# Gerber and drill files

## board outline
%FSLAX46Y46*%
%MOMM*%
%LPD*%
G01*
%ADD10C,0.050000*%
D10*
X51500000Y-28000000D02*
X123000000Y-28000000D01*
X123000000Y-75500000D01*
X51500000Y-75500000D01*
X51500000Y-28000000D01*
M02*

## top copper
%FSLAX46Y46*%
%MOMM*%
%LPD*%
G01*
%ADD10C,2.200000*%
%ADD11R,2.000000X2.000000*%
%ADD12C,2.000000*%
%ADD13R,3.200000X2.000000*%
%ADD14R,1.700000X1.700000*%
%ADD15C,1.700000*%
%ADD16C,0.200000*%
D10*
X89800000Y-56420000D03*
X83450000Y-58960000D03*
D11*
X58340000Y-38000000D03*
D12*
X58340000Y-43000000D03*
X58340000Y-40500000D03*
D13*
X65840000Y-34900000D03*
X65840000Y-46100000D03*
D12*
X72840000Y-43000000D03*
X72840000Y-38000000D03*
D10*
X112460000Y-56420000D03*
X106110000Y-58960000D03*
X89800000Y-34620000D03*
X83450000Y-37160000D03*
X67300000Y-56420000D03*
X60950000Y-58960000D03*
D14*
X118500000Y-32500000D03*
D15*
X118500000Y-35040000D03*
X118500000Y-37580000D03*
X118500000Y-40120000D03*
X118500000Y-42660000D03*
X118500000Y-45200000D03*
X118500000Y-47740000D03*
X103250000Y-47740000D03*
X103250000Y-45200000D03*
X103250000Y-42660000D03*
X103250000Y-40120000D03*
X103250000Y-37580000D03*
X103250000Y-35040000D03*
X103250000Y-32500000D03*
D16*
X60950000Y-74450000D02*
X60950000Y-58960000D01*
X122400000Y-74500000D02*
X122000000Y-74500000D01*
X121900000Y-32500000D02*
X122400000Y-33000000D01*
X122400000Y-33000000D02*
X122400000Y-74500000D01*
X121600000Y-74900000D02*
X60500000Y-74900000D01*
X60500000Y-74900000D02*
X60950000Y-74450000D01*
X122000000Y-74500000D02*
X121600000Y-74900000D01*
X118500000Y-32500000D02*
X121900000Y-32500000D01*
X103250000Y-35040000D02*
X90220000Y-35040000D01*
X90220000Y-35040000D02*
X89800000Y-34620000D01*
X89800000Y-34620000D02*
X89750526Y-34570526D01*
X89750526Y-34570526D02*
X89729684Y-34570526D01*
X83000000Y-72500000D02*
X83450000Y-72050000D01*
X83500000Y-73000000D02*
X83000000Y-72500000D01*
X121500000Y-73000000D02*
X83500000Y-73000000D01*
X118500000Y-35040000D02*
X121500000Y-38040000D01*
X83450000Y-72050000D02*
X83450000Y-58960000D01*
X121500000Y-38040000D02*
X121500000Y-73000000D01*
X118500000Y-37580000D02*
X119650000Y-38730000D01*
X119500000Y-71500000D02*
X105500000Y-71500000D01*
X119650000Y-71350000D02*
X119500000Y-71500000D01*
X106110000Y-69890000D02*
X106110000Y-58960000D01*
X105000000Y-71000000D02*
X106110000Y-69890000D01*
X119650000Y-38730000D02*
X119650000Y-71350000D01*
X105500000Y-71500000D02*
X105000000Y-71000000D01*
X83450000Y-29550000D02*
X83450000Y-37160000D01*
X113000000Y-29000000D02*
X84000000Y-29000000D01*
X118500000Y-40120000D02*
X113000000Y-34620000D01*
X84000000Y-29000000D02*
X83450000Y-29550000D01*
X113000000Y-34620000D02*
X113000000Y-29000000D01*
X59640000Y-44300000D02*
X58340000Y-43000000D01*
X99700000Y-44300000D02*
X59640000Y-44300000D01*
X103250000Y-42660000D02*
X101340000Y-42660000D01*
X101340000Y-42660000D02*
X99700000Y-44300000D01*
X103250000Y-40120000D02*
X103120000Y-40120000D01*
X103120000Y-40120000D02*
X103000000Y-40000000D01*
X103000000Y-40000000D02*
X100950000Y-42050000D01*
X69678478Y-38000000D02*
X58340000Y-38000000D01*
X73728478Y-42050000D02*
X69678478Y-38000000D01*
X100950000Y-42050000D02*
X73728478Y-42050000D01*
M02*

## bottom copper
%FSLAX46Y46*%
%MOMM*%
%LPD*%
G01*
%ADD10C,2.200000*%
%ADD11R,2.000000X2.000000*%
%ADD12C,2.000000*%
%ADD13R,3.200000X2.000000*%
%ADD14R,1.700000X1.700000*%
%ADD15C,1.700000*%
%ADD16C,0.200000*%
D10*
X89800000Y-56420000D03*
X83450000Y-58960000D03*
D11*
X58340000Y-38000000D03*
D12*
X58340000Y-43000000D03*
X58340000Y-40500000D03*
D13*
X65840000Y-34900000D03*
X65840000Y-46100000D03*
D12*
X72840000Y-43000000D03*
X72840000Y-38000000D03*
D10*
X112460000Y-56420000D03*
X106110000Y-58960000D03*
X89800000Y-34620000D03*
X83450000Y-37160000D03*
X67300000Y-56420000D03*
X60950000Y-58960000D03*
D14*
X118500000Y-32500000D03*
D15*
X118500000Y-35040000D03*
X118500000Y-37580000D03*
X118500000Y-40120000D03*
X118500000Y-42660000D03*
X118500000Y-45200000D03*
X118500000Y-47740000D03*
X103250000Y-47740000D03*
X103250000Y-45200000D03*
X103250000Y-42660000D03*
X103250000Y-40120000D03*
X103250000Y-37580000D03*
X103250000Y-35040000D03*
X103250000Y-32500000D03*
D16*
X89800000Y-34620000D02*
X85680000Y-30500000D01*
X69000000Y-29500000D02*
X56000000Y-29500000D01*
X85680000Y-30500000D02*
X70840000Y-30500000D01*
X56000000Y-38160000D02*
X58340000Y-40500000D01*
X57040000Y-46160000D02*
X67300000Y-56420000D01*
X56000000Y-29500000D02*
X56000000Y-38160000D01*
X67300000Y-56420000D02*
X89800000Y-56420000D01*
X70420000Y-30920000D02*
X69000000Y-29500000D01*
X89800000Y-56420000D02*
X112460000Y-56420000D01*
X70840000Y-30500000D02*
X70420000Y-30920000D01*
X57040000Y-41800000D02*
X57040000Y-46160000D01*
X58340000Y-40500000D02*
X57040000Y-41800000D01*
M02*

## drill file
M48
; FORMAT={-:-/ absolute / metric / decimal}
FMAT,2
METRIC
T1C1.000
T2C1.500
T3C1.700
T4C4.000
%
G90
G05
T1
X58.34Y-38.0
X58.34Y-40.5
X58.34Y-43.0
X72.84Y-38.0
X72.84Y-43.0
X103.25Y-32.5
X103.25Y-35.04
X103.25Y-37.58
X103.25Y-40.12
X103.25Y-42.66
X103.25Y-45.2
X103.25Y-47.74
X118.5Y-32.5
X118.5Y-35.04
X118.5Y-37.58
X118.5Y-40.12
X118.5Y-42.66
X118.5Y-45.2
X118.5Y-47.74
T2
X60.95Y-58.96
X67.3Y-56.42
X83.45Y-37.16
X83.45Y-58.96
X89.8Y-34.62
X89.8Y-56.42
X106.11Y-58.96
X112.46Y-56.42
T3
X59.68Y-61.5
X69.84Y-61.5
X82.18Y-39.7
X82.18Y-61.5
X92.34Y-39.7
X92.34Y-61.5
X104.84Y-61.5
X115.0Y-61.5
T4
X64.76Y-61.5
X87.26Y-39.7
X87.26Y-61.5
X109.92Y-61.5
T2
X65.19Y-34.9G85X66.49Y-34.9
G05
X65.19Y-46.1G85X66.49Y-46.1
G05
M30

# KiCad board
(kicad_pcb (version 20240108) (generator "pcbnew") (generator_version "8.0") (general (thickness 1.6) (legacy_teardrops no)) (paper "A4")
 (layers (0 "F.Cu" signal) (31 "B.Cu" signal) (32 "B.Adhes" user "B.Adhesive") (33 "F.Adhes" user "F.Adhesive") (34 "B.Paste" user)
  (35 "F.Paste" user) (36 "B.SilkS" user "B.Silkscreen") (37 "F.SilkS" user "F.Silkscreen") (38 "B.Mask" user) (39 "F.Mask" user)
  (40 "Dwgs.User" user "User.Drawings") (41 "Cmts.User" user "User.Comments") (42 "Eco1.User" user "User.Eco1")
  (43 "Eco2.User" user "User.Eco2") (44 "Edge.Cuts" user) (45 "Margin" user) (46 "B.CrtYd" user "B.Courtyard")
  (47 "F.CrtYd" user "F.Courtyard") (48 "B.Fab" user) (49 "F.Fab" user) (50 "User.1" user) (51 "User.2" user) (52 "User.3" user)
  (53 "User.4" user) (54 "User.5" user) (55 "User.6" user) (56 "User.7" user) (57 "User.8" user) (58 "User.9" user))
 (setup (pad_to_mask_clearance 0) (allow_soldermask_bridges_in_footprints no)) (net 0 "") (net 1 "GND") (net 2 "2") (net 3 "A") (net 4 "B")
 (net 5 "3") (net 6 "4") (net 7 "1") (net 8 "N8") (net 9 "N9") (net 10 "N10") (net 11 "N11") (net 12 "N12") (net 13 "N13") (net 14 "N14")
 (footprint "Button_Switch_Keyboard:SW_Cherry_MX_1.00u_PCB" (layer "F.Cu") (at 89.8 56.42)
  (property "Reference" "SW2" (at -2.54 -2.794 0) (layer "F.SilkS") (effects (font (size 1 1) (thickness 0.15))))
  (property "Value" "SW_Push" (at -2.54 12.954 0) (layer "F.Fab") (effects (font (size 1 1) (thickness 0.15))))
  (pad "" np_thru_hole circle (at -7.62 5.08) (size 1.7 1.7) (drill 1.7) (layers "*.Cu" "*.Mask"))
  (pad "" np_thru_hole circle (at -2.54 5.08) (size 4 4) (drill 4) (layers "*.Cu" "*.Mask"))
  (pad "" np_thru_hole circle (at 2.54 5.08) (size 1.7 1.7) (drill 1.7) (layers "*.Cu" "*.Mask"))
  (pad "1" thru_hole circle (at 0 0) (size 2.2 2.2) (drill 1.5) (layers "*.Cu" "*.Mask") (remove_unused_layers no) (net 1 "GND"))
  (pad "2" thru_hole circle (at -6.35 2.54) (size 2.2 2.2) (drill 1.5) (layers "*.Cu" "*.Mask") (remove_unused_layers no) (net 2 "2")))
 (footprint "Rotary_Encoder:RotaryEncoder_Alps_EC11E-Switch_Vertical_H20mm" (layer "F.Cu") (at 58.34 38)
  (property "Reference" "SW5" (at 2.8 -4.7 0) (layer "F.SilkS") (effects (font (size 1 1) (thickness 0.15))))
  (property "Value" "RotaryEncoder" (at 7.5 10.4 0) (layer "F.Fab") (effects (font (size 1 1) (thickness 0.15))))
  (pad "A" thru_hole rect (at 0 0) (size 2 2) (drill 1) (layers "*.Cu" "*.Mask") (remove_unused_layers no) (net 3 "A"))
  (pad "B" thru_hole circle (at 0 5) (size 2 2) (drill 1) (layers "*.Cu" "*.Mask") (remove_unused_layers no) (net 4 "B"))
  (pad "C" thru_hole circle (at 0 2.5) (size 2 2) (drill 1) (layers "*.Cu" "*.Mask") (remove_unused_layers no) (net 1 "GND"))
  (pad "MP" thru_hole rect (at 7.5 -3.1) (size 3.2 2) (drill oval 2.8 1.5) (layers "*.Cu" "*.Mask") (remove_unused_layers no))
  (pad "MP" thru_hole rect (at 7.5 8.1) (size 3.2 2) (drill oval 2.8 1.5) (layers "*.Cu" "*.Mask") (remove_unused_layers no))
  (pad "S1" thru_hole circle (at 14.5 5) (size 2 2) (drill 1) (layers "*.Cu" "*.Mask") (remove_unused_layers no))
  (pad "S2" thru_hole circle (at 14.5 0) (size 2 2) (drill 1) (layers "*.Cu" "*.Mask") (remove_unused_layers no)))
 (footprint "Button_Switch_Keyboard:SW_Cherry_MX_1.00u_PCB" (layer "F.Cu") (at 112.46 56.42)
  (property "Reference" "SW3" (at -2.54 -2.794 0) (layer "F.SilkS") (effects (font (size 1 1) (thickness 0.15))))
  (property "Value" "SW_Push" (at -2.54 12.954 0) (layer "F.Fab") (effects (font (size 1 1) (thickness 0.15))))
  (pad "" np_thru_hole circle (at -7.62 5.08) (size 1.7 1.7) (drill 1.7) (layers "*.Cu" "*.Mask"))
  (pad "" np_thru_hole circle (at -2.54 5.08) (size 4 4) (drill 4) (layers "*.Cu" "*.Mask"))
  (pad "" np_thru_hole circle (at 2.54 5.08) (size 1.7 1.7) (drill 1.7) (layers "*.Cu" "*.Mask"))
  (pad "1" thru_hole circle (at 0 0) (size 2.2 2.2) (drill 1.5) (layers "*.Cu" "*.Mask") (remove_unused_layers no) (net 1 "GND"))
  (pad "2" thru_hole circle (at -6.35 2.54) (size 2.2 2.2) (drill 1.5) (layers "*.Cu" "*.Mask") (remove_unused_layers no) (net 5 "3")))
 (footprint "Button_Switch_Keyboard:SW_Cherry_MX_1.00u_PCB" (layer "F.Cu") (at 89.8 34.62)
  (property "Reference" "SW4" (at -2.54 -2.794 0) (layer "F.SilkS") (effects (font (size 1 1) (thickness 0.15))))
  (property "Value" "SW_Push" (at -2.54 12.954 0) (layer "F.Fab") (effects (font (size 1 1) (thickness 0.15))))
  (pad "" np_thru_hole circle (at -7.62 5.08) (size 1.7 1.7) (drill 1.7) (layers "*.Cu" "*.Mask"))
  (pad "" np_thru_hole circle (at -2.54 5.08) (size 4 4) (drill 4) (layers "*.Cu" "*.Mask"))
  (pad "" np_thru_hole circle (at 2.54 5.08) (size 1.7 1.7) (drill 1.7) (layers "*.Cu" "*.Mask"))
  (pad "1" thru_hole circle (at 0 0) (size 2.2 2.2) (drill 1.5) (layers "*.Cu" "*.Mask") (remove_unused_layers no) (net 1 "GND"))
  (pad "2" thru_hole circle (at -6.35 2.54) (size 2.2 2.2) (drill 1.5) (layers "*.Cu" "*.Mask") (remove_unused_layers no) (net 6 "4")))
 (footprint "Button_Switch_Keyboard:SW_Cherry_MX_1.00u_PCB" (layer "F.Cu") (at 67.3 56.42)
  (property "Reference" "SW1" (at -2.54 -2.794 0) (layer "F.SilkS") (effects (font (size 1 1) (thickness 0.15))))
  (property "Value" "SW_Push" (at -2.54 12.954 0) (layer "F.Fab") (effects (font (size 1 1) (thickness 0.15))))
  (pad "" np_thru_hole circle (at -7.62 5.08) (size 1.7 1.7) (drill 1.7) (layers "*.Cu" "*.Mask"))
  (pad "" np_thru_hole circle (at -2.54 5.08) (size 4 4) (drill 4) (layers "*.Cu" "*.Mask"))
  (pad "" np_thru_hole circle (at 2.54 5.08) (size 1.7 1.7) (drill 1.7) (layers "*.Cu" "*.Mask"))
  (pad "1" thru_hole circle (at 0 0) (size 2.2 2.2) (drill 1.5) (layers "*.Cu" "*.Mask") (remove_unused_layers no) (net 1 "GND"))
  (pad "2" thru_hole circle (at -6.35 2.54) (size 2.2 2.2) (drill 1.5) (layers "*.Cu" "*.Mask") (remove_unused_layers no) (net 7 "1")))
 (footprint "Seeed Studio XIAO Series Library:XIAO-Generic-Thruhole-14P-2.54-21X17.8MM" (layer "B.Cu") (at 110.875 40.12 180)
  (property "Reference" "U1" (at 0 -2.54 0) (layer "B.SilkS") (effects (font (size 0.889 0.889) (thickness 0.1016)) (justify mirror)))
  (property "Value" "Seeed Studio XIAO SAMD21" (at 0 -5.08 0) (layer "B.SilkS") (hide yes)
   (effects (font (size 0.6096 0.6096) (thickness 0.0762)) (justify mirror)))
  (pad "1" thru_hole rect (at -7.625 7.62 180) (size 1.7 1.7) (drill 1) (layers "*.Cu" "*.Mask") (remove_unused_layers no) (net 7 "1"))
  (pad "2" thru_hole circle (at -7.625 5.08 180) (size 1.7 1.7) (drill 1) (layers "*.Cu" "*.Mask") (remove_unused_layers no) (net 2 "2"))
  (pad "3" thru_hole circle (at -7.625 2.54 180) (size 1.7 1.7) (drill 1) (layers "*.Cu" "*.Mask") (remove_unused_layers no) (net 5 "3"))
  (pad "4" thru_hole circle (at -7.625 0 180) (size 1.7 1.7) (drill 1) (layers "*.Cu" "*.Mask") (remove_unused_layers no) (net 6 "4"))
  (pad "5" thru_hole circle (at -7.625 -2.54 180) (size 1.7 1.7) (drill 1) (layers "*.Cu" "*.Mask") (remove_unused_layers no) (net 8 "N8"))
  (pad "6" thru_hole circle (at -7.625 -5.08) (size 1.7 1.7) (drill 1) (layers "*.Cu" "*.Mask") (remove_unused_layers no) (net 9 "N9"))
  (pad "7" thru_hole circle (at -7.625 -7.62 180) (size 1.7 1.7) (drill 1) (layers "*.Cu" "*.Mask") (remove_unused_layers no) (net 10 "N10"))
  (pad "8" thru_hole circle (at 7.625 -7.62 180) (size 1.7 1.7) (drill 1) (layers "*.Cu" "*.Mask") (remove_unused_layers no) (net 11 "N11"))
  (pad "9" thru_hole circle (at 7.625 -5.08 180) (size 1.7 1.7) (drill 1) (layers "*.Cu" "*.Mask") (remove_unused_layers no) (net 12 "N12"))
  (pad "10" thru_hole circle (at 7.625 -2.54 180) (size 1.7 1.7) (drill 1) (layers "*.Cu" "*.Mask") (remove_unused_layers no) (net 4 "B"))
  (pad "11" thru_hole circle (at 7.625 0 180) (size 1.7 1.7) (drill 1) (layers "*.Cu" "*.Mask") (remove_unused_layers no) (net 3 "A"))
  (pad "12" thru_hole circle (at 7.625 2.54 180) (size 1.7 1.7) (drill 1) (layers "*.Cu" "*.Mask") (remove_unused_layers no) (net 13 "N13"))
  (pad "13" thru_hole circle (at 7.625 5.08 180) (size 1.7 1.7) (drill 1) (layers "*.Cu" "*.Mask") (remove_unused_layers no) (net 1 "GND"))
  (pad "14" thru_hole circle (at 7.625 7.62 180) (size 1.7 1.7) (drill 1) (layers "*.Cu" "*.Mask") (remove_unused_layers no) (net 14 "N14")))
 (gr_rect (start 51.5 28) (end 123 75.5) (stroke (width 0.05) (type default)) (fill none) (layer "Edge.Cuts"))
 (segment (start 60.95 74.45) (end 60.95 58.96) (width 0.2) (layer "F.Cu") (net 7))
 (segment (start 122.4 74.5) (end 122 74.5) (width 0.2) (layer "F.Cu") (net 7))
 (segment (start 121.9 32.5) (end 122.4 33) (width 0.2) (layer "F.Cu") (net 7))
 (segment (start 122.4 33) (end 122.4 74.5) (width 0.2) (layer "F.Cu") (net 7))
 (segment (start 121.6 74.9) (end 60.5 74.9) (width 0.2) (layer "F.Cu") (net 7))
 (segment (start 60.5 74.9) (end 60.95 74.45) (width 0.2) (layer "F.Cu") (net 7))
 (segment (start 122 74.5) (end 121.6 74.9) (width 0.2) (layer "F.Cu") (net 7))
 (segment (start 118.5 32.5) (end 121.9 32.5) (width 0.2) (layer "F.Cu") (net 7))
 (segment (start 103.25 35.04) (end 90.22 35.04) (width 0.2) (layer "F.Cu") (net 1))
 (segment (start 90.22 35.04) (end 89.8 34.62) (width 0.2) (layer "F.Cu") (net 1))
 (segment (start 89.8 34.62) (end 89.750526 34.570526) (width 0.2) (layer "F.Cu") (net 1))
 (segment (start 89.750526 34.570526) (end 89.729684 34.570526) (width 0.2) (layer "F.Cu") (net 1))
 (segment (start 89.8 34.62) (end 85.68 30.5) (width 0.2) (layer "B.Cu") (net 1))
 (segment (start 69 29.5) (end 56 29.5) (width 0.2) (layer "B.Cu") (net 1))
 (segment (start 85.68 30.5) (end 70.84 30.5) (width 0.2) (layer "B.Cu") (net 1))
 (segment (start 56 38.16) (end 58.34 40.5) (width 0.2) (layer "B.Cu") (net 1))
 (segment (start 57.04 46.16) (end 67.3 56.42) (width 0.2) (layer "B.Cu") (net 1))
 (segment (start 56 29.5) (end 56 38.16) (width 0.2) (layer "B.Cu") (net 1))
 (segment (start 67.3 56.42) (end 89.8 56.42) (width 0.2) (layer "B.Cu") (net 1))
 (segment (start 70.42 30.92) (end 69 29.5) (width 0.2) (layer "B.Cu") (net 1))
 (segment (start 89.8 56.42) (end 112.46 56.42) (width 0.2) (layer "B.Cu") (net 1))
 (segment (start 70.84 30.5) (end 70.42 30.92) (width 0.2) (layer "B.Cu") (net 1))
 (segment (start 57.04 41.8) (end 57.04 46.16) (width 0.2) (layer "B.Cu") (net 1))
 (segment (start 58.34 40.5) (end 57.04 41.8) (width 0.2) (layer "B.Cu") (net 1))
 (segment (start 83 72.5) (end 83.45 72.05) (width 0.2) (layer "F.Cu") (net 2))
 (segment (start 83.5 73) (end 83 72.5) (width 0.2) (layer "F.Cu") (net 2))
 (segment (start 121.5 73) (end 83.5 73) (width 0.2) (layer "F.Cu") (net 2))
 (segment (start 118.5 35.04) (end 121.5 38.04) (width 0.2) (layer "F.Cu") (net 2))
 (segment (start 83.45 72.05) (end 83.45 58.96) (width 0.2) (layer "F.Cu") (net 2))
 (segment (start 121.5 38.04) (end 121.5 73) (width 0.2) (layer "F.Cu") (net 2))
 (segment (start 118.5 37.58) (end 119.65 38.73) (width 0.2) (layer "F.Cu") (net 5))
 (segment (start 119.5 71.5) (end 105.5 71.5) (width 0.2) (layer "F.Cu") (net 5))
 (segment (start 119.65 71.35) (end 119.5 71.5) (width 0.2) (layer "F.Cu") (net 5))
 (segment (start 106.11 69.89) (end 106.11 58.96) (width 0.2) (layer "F.Cu") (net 5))
 (segment (start 105 71) (end 106.11 69.89) (width 0.2) (layer "F.Cu") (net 5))
 (segment (start 119.65 38.73) (end 119.65 71.35) (width 0.2) (layer "F.Cu") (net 5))
 (segment (start 105.5 71.5) (end 105 71) (width 0.2) (layer "F.Cu") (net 5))
 (segment (start 83.45 29.55) (end 83.45 37.16) (width 0.2) (layer "F.Cu") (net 6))
 (segment (start 113 29) (end 84 29) (width 0.2) (layer "F.Cu") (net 6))
 (segment (start 118.5 40.12) (end 113 34.62) (width 0.2) (layer "F.Cu") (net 6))
 (segment (start 84 29) (end 83.45 29.55) (width 0.2) (layer "F.Cu") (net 6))
 (segment (start 113 34.62) (end 113 29) (width 0.2) (layer "F.Cu") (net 6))
 (segment (start 59.64 44.3) (end 58.34 43) (width 0.2) (layer "F.Cu") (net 4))
 (segment (start 99.7 44.3) (end 59.64 44.3) (width 0.2) (layer "F.Cu") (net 4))
 (segment (start 103.25 42.66) (end 101.34 42.66) (width 0.2) (layer "F.Cu") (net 4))
 (segment (start 101.34 42.66) (end 99.7 44.3) (width 0.2) (layer "F.Cu") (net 4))
 (segment (start 103.25 40.12) (end 103.12 40.12) (width 0.2) (layer "F.Cu") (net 3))
 (segment (start 103.12 40.12) (end 103 40) (width 0.2) (layer "F.Cu") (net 3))
 (segment (start 103 40) (end 100.95 42.05) (width 0.2) (layer "F.Cu") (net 3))
 (segment (start 69.678478 38) (end 58.34 38) (width 0.2) (layer "F.Cu") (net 3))
 (segment (start 73.728478 42.05) (end 69.678478 38) (width 0.2) (layer "F.Cu") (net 3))
 (segment (start 100.95 42.05) (end 73.728478 42.05) (width 0.2) (layer "F.Cu") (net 3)))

